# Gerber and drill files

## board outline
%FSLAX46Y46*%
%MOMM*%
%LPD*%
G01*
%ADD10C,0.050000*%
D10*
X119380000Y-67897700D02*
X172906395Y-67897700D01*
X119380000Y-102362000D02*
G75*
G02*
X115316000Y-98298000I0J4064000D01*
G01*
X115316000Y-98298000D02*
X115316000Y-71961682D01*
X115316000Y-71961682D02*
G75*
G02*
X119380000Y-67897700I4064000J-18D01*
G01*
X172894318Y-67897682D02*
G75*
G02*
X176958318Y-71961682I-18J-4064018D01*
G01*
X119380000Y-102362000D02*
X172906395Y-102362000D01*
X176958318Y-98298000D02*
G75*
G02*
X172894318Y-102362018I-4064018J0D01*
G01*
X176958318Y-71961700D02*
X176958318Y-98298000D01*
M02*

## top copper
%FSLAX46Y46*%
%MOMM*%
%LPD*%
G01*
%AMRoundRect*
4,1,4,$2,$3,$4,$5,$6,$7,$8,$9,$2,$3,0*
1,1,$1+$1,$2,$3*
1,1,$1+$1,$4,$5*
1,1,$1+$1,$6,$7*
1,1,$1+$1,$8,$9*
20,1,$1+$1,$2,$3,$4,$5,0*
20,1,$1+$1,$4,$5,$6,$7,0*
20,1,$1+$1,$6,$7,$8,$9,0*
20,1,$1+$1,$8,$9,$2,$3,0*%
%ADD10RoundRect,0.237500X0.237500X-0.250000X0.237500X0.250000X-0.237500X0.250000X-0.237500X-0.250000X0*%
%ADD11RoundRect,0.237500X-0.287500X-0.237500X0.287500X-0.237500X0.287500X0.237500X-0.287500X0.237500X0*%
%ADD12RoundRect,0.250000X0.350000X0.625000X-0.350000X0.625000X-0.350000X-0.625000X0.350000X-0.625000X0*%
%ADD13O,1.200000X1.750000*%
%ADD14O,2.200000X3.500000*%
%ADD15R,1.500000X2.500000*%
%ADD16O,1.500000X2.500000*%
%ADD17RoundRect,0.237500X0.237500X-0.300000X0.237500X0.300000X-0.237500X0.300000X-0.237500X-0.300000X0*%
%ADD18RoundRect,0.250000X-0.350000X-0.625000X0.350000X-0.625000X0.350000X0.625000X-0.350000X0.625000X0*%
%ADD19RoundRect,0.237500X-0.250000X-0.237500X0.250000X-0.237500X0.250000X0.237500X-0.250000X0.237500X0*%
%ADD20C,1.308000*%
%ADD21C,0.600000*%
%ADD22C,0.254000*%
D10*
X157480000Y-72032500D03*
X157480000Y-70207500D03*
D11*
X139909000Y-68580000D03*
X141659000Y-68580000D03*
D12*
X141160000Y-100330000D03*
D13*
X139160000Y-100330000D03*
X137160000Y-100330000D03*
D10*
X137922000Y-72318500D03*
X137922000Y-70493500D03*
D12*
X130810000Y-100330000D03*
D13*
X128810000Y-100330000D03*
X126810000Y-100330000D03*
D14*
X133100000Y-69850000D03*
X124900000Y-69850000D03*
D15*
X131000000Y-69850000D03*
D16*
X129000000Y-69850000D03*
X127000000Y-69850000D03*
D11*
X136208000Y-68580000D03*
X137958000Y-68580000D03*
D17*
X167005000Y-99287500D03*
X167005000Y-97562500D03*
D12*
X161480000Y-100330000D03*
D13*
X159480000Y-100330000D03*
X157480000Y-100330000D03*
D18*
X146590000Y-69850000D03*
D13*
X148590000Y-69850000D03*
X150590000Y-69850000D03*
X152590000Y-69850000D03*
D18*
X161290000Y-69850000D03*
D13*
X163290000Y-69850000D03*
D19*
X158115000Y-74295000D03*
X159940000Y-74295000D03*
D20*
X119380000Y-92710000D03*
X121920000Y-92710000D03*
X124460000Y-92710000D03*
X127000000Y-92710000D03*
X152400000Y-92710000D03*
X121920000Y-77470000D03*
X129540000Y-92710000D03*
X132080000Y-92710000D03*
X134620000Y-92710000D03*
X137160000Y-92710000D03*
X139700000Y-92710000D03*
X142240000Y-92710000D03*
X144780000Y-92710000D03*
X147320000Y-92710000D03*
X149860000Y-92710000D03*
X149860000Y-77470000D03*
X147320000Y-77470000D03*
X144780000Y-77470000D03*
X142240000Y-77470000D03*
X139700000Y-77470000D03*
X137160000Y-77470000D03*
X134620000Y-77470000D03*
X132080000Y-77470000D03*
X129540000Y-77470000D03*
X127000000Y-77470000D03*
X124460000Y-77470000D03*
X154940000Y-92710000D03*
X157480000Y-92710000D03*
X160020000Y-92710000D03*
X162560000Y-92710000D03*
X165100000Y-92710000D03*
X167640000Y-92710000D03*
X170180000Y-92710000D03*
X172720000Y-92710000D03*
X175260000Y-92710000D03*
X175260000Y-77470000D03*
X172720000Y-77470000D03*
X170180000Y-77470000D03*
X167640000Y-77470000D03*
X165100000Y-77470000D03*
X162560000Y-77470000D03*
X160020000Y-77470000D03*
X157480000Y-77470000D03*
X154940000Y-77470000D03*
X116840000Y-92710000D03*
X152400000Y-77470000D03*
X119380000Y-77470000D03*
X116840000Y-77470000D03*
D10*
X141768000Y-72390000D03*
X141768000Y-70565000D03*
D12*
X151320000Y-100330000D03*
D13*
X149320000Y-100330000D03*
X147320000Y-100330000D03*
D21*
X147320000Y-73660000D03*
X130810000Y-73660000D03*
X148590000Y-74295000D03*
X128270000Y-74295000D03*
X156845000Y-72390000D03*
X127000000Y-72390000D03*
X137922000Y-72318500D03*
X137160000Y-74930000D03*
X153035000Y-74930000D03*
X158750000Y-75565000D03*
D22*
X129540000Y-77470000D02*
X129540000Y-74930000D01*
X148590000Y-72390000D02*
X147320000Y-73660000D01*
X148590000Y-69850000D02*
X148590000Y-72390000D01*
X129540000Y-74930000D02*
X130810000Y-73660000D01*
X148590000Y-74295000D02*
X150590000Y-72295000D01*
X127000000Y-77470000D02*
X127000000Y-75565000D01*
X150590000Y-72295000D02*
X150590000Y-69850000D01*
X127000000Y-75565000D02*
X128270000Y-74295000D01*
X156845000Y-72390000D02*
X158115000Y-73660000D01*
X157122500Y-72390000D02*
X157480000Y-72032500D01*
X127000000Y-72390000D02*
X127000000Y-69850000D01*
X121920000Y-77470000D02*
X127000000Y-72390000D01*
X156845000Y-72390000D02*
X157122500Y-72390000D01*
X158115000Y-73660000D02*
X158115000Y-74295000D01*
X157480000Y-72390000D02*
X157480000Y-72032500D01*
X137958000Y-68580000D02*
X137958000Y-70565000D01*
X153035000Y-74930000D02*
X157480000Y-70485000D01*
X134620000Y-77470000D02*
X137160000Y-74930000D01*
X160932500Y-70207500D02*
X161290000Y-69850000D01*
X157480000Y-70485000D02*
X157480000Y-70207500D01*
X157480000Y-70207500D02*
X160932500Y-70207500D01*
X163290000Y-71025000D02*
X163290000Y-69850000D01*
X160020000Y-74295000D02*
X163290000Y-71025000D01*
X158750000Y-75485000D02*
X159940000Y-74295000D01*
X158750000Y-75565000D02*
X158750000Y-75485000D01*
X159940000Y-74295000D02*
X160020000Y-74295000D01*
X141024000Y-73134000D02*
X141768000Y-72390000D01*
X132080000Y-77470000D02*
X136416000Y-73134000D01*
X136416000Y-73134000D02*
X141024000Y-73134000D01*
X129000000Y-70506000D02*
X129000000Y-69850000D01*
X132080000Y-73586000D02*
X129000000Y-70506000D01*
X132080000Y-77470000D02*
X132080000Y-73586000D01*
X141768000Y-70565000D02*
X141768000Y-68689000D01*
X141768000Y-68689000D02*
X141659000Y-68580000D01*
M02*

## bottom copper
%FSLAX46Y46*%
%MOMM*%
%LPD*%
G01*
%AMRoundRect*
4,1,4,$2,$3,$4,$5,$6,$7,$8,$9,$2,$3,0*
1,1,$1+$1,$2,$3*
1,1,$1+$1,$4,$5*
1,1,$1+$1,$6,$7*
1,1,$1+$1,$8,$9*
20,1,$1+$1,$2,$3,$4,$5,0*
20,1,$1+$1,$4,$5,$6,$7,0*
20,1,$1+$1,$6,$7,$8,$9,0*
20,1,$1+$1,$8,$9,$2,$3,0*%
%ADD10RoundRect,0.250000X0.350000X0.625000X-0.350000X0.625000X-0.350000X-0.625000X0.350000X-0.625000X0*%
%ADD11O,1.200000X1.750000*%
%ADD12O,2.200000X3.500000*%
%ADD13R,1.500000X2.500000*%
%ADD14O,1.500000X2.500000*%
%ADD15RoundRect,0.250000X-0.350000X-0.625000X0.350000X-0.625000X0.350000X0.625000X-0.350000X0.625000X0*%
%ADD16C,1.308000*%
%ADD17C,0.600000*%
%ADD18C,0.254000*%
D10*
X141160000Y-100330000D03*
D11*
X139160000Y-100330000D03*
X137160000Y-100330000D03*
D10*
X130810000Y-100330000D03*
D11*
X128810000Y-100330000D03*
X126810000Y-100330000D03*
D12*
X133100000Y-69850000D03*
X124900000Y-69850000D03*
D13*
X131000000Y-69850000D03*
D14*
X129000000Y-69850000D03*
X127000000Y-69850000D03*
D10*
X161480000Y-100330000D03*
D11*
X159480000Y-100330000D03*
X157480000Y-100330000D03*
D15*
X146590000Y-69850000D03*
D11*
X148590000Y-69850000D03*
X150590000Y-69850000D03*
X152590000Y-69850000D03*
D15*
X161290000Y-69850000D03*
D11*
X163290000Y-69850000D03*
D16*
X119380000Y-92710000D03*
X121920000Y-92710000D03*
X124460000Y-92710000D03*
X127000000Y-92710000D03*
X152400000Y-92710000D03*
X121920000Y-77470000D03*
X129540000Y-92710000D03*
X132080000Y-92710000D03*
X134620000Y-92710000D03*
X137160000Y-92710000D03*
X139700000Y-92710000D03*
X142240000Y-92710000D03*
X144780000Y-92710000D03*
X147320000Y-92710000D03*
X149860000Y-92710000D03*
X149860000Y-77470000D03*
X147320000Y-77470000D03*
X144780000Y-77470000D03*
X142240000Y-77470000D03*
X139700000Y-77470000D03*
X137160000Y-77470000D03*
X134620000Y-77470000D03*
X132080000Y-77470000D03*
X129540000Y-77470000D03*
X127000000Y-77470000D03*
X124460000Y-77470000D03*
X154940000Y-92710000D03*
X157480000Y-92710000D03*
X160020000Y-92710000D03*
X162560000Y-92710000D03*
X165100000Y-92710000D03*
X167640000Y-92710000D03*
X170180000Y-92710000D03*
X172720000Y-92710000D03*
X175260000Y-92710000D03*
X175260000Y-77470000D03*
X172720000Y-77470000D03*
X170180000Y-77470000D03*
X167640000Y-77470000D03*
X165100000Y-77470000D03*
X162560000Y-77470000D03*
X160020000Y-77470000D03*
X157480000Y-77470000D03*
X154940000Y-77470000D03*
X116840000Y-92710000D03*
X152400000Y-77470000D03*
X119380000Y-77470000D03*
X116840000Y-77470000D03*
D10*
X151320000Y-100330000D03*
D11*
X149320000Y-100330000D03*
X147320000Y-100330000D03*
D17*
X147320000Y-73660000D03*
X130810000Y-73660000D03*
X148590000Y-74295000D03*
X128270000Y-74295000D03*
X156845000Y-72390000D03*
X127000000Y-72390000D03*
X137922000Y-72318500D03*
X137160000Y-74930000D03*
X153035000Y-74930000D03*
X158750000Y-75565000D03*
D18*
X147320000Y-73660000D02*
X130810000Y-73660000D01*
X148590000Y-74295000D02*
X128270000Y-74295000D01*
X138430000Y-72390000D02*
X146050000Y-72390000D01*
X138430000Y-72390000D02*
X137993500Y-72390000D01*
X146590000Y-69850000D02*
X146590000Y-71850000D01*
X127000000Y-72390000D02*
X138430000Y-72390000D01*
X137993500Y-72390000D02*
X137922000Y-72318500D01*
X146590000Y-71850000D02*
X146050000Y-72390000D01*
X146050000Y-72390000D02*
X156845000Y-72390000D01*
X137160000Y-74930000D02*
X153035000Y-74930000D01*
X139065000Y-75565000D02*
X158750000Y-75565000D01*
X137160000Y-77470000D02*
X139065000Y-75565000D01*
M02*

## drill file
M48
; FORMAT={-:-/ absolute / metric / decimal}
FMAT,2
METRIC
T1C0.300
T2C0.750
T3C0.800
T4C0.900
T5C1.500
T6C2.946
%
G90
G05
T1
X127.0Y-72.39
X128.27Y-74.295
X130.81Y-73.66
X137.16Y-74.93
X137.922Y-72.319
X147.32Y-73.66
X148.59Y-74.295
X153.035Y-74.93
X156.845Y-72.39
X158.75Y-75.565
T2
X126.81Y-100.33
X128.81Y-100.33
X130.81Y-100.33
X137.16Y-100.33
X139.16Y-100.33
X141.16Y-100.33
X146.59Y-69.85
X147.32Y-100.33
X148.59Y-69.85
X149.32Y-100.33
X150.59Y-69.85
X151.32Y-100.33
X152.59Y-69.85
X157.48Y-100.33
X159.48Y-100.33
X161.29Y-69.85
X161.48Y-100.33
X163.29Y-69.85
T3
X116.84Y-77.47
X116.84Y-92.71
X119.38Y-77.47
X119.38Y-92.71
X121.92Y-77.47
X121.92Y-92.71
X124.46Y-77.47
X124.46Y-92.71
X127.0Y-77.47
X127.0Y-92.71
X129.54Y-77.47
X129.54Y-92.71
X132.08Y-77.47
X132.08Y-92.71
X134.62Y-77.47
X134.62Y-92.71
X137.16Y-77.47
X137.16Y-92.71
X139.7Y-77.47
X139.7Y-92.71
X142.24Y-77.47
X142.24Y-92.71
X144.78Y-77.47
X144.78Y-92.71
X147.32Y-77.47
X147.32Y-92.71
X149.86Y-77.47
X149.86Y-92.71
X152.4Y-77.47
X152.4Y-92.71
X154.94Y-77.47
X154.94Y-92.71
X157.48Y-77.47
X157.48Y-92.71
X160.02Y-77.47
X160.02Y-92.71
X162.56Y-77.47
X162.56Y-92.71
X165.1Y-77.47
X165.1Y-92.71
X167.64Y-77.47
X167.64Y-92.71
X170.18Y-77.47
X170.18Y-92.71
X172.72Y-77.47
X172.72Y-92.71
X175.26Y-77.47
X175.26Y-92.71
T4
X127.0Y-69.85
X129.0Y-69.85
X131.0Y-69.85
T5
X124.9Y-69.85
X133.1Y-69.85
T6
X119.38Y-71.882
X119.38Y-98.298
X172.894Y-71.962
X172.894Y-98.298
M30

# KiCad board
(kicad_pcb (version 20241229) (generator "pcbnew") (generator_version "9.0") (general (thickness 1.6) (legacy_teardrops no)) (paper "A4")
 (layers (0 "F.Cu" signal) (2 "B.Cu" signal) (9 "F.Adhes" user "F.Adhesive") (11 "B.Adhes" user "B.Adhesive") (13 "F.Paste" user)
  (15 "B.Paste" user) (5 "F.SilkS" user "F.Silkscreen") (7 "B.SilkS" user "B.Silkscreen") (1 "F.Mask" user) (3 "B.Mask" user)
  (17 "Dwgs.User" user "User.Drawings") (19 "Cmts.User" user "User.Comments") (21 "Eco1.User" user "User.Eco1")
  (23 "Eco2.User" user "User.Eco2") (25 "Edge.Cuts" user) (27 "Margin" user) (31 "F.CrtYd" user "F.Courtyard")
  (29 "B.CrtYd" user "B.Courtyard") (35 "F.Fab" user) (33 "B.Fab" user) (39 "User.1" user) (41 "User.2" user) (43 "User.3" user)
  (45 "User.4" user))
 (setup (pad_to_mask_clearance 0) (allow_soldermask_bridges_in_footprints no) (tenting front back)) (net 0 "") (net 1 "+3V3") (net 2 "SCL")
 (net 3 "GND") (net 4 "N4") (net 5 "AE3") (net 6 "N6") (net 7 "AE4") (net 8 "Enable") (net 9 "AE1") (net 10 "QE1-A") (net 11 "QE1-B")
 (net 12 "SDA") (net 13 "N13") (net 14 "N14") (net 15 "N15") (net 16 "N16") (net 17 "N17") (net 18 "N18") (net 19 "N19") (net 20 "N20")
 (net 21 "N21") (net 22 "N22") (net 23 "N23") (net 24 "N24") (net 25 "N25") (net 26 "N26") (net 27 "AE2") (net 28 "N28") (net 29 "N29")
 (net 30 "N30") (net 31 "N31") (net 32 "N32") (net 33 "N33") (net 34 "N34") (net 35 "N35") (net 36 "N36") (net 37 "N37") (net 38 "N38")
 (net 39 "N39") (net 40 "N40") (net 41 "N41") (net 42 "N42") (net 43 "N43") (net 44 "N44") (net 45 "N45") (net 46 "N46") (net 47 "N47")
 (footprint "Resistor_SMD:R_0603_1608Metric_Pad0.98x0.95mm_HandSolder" (layer "F.Cu") (at 157.48 71.12 90)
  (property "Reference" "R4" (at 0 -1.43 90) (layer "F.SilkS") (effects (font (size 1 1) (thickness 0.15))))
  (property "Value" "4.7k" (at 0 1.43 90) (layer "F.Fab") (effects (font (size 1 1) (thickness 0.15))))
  (pad "1" smd roundrect (at -0.9125 0 90) (size 0.975 0.95) (layers "F.Cu" "F.Mask" "F.Paste") (roundrect_rratio 0.25) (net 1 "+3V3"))
  (pad "2" smd roundrect (at 0.9125 0 90) (size 0.975 0.95) (layers "F.Cu" "F.Mask" "F.Paste") (roundrect_rratio 0.25) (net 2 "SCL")))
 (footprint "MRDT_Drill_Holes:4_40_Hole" (layer "F.Cu") (at 172.894318 98.298)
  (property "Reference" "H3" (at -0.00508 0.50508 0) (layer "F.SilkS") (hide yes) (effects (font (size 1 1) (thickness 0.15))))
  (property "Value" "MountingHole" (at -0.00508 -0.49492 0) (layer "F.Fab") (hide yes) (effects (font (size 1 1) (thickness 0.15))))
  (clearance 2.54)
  (pad "" np_thru_hole circle (at 0 0) (size 2.9464 2.9464) (drill 2.9464) (layers "*.Cu" "*.Mask") (clearance 2.5)))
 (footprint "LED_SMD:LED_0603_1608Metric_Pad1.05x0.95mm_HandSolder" (layer "F.Cu") (at 140.784 68.58)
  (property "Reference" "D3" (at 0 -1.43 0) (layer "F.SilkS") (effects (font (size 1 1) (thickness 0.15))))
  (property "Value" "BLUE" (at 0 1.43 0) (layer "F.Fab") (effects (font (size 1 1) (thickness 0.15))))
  (pad "1" smd roundrect (at -0.875 0) (size 1.05 0.95) (layers "F.Cu" "F.Mask" "F.Paste") (roundrect_rratio 0.25) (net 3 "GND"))
  (pad "2" smd roundrect (at 0.875 0) (size 1.05 0.95) (layers "F.Cu" "F.Mask" "F.Paste") (roundrect_rratio 0.25) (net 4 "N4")))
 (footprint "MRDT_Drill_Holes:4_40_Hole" (layer "F.Cu") (at 119.38 71.882)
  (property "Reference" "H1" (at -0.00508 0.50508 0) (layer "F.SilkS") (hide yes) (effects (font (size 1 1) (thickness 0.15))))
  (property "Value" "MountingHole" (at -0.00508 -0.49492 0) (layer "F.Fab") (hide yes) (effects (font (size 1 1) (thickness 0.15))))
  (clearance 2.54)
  (pad "" np_thru_hole circle (at 0 0) (size 2.9464 2.9464) (drill 2.9464) (layers "*.Cu" "*.Mask") (clearance 2.5)))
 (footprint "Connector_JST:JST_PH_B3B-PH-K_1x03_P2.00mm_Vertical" (layer "F.Cu") (at 141.16 100.33 180)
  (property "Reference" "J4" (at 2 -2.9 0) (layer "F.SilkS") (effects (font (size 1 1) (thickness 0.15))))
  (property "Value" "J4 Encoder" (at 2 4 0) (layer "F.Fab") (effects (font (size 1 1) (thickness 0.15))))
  (pad "1" thru_hole roundrect (at 0 0 180) (size 1.2 1.75) (drill 0.75) (layers "*.Cu" "*.Mask") (remove_unused_layers no)
   (roundrect_rratio 0.208333) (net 1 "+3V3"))
  (pad "2" thru_hole oval (at 2 0 180) (size 1.2 1.75) (drill 0.75) (layers "*.Cu" "*.Mask") (remove_unused_layers no) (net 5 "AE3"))
  (pad "3" thru_hole oval (at 4 0 180) (size 1.2 1.75) (drill 0.75) (layers "*.Cu" "*.Mask") (remove_unused_layers no) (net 3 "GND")))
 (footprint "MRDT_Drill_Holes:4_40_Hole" (layer "F.Cu") (at 119.38 98.298)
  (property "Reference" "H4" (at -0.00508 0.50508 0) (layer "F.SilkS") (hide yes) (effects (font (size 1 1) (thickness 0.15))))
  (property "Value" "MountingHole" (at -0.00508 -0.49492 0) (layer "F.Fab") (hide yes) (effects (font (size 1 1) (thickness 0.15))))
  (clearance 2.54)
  (pad "" np_thru_hole circle (at 0 0) (size 2.9464 2.9464) (drill 2.9464) (layers "*.Cu" "*.Mask") (clearance 2.5)))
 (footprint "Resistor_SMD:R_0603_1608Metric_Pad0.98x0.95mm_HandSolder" (layer "F.Cu") (at 137.922 71.406 90)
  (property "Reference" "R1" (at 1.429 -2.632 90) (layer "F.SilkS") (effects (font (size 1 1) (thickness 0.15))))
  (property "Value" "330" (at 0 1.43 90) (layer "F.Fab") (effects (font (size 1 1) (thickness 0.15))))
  (pad "1" smd roundrect (at -0.9125 0 90) (size 0.975 0.95) (layers "F.Cu" "F.Mask" "F.Paste") (roundrect_rratio 0.25) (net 1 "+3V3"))
  (pad "2" smd roundrect (at 0.9125 0 90) (size 0.975 0.95) (layers "F.Cu" "F.Mask" "F.Paste") (roundrect_rratio 0.25) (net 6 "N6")))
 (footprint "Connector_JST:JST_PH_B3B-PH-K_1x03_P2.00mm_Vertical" (layer "F.Cu") (at 130.81 100.33 180)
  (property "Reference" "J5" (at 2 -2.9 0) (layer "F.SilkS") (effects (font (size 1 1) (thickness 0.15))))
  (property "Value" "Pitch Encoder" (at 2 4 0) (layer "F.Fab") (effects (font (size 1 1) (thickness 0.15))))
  (pad "1" thru_hole roundrect (at 0 0 180) (size 1.2 1.75) (drill 0.75) (layers "*.Cu" "*.Mask") (remove_unused_layers no)
   (roundrect_rratio 0.208333) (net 1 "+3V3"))
  (pad "2" thru_hole oval (at 2 0 180) (size 1.2 1.75) (drill 0.75) (layers "*.Cu" "*.Mask") (remove_unused_layers no) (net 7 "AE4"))
  (pad "3" thru_hole oval (at 4 0 180) (size 1.2 1.75) (drill 0.75) (layers "*.Cu" "*.Mask") (remove_unused_layers no) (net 3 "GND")))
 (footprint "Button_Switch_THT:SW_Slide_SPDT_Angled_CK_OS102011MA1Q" (layer "F.Cu") (at 131 69.85 180)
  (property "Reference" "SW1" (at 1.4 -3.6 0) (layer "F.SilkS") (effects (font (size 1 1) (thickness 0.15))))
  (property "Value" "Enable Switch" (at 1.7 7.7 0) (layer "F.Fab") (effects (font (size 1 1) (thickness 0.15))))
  (pad "" thru_hole oval (at -2.1 0 180) (size 2.2 3.5) (drill 1.5) (layers "*.Cu" "*.Mask") (remove_unused_layers no))
  (pad "" thru_hole oval (at 6.1 0 180) (size 2.2 3.5) (drill 1.5) (layers "*.Cu" "*.Mask") (remove_unused_layers no))
  (pad "1" thru_hole rect (at 0 0 180) (size 1.5 2.5) (drill 0.9) (layers "*.Cu" "*.Mask") (remove_unused_layers no) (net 3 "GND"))
  (pad "2" thru_hole oval (at 2 0 180) (size 1.5 2.5) (drill 0.9) (layers "*.Cu" "*.Mask") (remove_unused_layers no) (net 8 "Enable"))
  (pad "3" thru_hole oval (at 4 0 180) (size 1.5 2.5) (drill 0.9) (layers "*.Cu" "*.Mask") (remove_unused_layers no) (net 1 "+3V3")))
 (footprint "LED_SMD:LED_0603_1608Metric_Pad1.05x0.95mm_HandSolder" (layer "F.Cu") (at 137.083 68.58)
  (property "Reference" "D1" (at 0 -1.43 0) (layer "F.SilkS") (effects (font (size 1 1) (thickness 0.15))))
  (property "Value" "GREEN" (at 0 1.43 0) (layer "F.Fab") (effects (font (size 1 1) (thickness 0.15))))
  (pad "1" smd roundrect (at -0.875 0) (size 1.05 0.95) (layers "F.Cu" "F.Mask" "F.Paste") (roundrect_rratio 0.25) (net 3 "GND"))
  (pad "2" smd roundrect (at 0.875 0) (size 1.05 0.95) (layers "F.Cu" "F.Mask" "F.Paste") (roundrect_rratio 0.25) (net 6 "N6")))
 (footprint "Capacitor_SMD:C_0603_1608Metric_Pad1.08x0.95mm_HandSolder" (layer "F.Cu") (at 167.005 98.425 90)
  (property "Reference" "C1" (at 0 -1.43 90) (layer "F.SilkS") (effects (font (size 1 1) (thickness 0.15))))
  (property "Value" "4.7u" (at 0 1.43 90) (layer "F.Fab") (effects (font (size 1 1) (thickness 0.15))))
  (pad "1" smd roundrect (at -0.8625 0 90) (size 1.075 0.95) (layers "F.Cu" "F.Mask" "F.Paste") (roundrect_rratio 0.25) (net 1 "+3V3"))
  (pad "2" smd roundrect (at 0.8625 0 90) (size 1.075 0.95) (layers "F.Cu" "F.Mask" "F.Paste") (roundrect_rratio 0.25) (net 3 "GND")))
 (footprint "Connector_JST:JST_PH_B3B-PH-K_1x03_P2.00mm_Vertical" (layer "F.Cu") (at 161.48 100.33 180)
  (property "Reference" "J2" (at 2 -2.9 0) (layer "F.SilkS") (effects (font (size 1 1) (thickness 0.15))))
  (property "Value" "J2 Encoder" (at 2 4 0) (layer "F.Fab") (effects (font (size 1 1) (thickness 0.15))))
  (pad "1" thru_hole roundrect (at 0 0 180) (size 1.2 1.75) (drill 0.75) (layers "*.Cu" "*.Mask") (remove_unused_layers no)
   (roundrect_rratio 0.208333) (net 1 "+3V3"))
  (pad "2" thru_hole oval (at 2 0 180) (size 1.2 1.75) (drill 0.75) (layers "*.Cu" "*.Mask") (remove_unused_layers no) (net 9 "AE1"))
  (pad "3" thru_hole oval (at 4 0 180) (size 1.2 1.75) (drill 0.75) (layers "*.Cu" "*.Mask") (remove_unused_layers no) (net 3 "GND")))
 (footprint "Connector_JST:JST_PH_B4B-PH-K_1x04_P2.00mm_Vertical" (layer "F.Cu") (at 146.59 69.85)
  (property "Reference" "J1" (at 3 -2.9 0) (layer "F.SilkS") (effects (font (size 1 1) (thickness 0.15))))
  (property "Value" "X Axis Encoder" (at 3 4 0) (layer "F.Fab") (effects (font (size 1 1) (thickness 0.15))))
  (pad "1" thru_hole roundrect (at 0 0) (size 1.2 1.75) (drill 0.75) (layers "*.Cu" "*.Mask") (remove_unused_layers no)
   (roundrect_rratio 0.208333) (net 1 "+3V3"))
  (pad "2" thru_hole oval (at 2 0) (size 1.2 1.75) (drill 0.75) (layers "*.Cu" "*.Mask") (remove_unused_layers no) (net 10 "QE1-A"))
  (pad "3" thru_hole oval (at 4 0) (size 1.2 1.75) (drill 0.75) (layers "*.Cu" "*.Mask") (remove_unused_layers no) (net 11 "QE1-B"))
  (pad "4" thru_hole oval (at 6 0) (size 1.2 1.75) (drill 0.75) (layers "*.Cu" "*.Mask") (remove_unused_layers no) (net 3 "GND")))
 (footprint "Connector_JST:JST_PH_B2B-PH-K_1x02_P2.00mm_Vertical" (layer "F.Cu") (at 161.29 69.85)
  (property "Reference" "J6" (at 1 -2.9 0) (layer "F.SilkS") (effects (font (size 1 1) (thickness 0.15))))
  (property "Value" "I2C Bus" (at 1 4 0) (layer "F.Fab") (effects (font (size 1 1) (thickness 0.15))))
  (pad "1" thru_hole roundrect (at 0 0) (size 1.2 1.75) (drill 0.75) (layers "*.Cu" "*.Mask") (remove_unused_layers no)
   (roundrect_rratio 0.208333) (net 2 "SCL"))
  (pad "2" thru_hole oval (at 2 0) (size 1.2 1.75) (drill 0.75) (layers "*.Cu" "*.Mask") (remove_unused_layers no) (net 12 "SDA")))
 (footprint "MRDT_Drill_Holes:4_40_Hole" (layer "F.Cu") (at 172.894318 71.961682)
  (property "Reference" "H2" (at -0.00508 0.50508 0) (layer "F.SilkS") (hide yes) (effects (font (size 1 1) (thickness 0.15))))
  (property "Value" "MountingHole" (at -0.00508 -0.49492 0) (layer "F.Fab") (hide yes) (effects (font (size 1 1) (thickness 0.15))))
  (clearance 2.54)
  (pad "" np_thru_hole circle (at 0 0) (size 2.9464 2.9464) (drill 2.9464) (layers "*.Cu" "*.Mask") (clearance 2.5)))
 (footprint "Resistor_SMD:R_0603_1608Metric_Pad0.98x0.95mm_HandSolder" (layer "F.Cu") (at 159.0275 74.295)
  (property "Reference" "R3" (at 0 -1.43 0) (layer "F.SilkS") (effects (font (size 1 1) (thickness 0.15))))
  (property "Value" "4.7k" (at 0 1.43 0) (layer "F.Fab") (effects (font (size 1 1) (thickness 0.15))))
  (pad "1" smd roundrect (at -0.9125 0) (size 0.975 0.95) (layers "F.Cu" "F.Mask" "F.Paste") (roundrect_rratio 0.25) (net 1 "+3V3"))
  (pad "2" smd roundrect (at 0.9125 0) (size 0.975 0.95) (layers "F.Cu" "F.Mask" "F.Paste") (roundrect_rratio 0.25) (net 12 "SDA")))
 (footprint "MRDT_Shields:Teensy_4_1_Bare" (layer "F.Cu") (at 146.05 85.09)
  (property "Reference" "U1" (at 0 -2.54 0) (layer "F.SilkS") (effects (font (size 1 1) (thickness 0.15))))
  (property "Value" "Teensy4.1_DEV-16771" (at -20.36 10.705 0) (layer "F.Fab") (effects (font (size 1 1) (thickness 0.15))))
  (pad "0" thru_hole circle (at -26.67 7.62) (size 1.308 1.308) (drill 0.8) (layers "*.Cu" "*.Mask") (remove_unused_layers no)
   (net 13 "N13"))
  (pad "1" thru_hole circle (at -24.13 7.62) (size 1.308 1.308) (drill 0.8) (layers "*.Cu" "*.Mask") (remove_unused_layers no)
   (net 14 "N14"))
  (pad "2" thru_hole circle (at -21.59 7.62) (size 1.308 1.308) (drill 0.8) (layers "*.Cu" "*.Mask") (remove_unused_layers no)
   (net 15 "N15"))
  (pad "3" thru_hole circle (at -19.05 7.62) (size 1.308 1.308) (drill 0.8) (layers "*.Cu" "*.Mask") (remove_unused_layers no)
   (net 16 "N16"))
  (pad "3.3V_1" thru_hole circle (at 6.35 7.62) (size 1.308 1.308) (drill 0.8) (layers "*.Cu" "*.Mask") (remove_unused_layers no)
   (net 1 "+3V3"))
  (pad "3.3V_2" thru_hole circle (at -24.13 -7.62) (size 1.308 1.308) (drill 0.8) (layers "*.Cu" "*.Mask") (remove_unused_layers no)
   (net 1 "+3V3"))
  (pad "4" thru_hole circle (at -16.51 7.62) (size 1.308 1.308) (drill 0.8) (layers "*.Cu" "*.Mask") (remove_unused_layers no)
   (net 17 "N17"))
  (pad "5" thru_hole circle (at -13.97 7.62) (size 1.308 1.308) (drill 0.8) (layers "*.Cu" "*.Mask") (remove_unused_layers no)
   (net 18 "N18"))
  (pad "6" thru_hole circle (at -11.43 7.62) (size 1.308 1.308) (drill 0.8) (layers "*.Cu" "*.Mask") (remove_unused_layers no)
   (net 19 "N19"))
  (pad "7" thru_hole circle (at -8.89 7.62) (size 1.308 1.308) (drill 0.8) (layers "*.Cu" "*.Mask") (remove_unused_layers no) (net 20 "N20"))
  (pad "8" thru_hole circle (at -6.35 7.62) (size 1.308 1.308) (drill 0.8) (layers "*.Cu" "*.Mask") (remove_unused_layers no) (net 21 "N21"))
  (pad "9" thru_hole circle (at -3.81 7.62) (size 1.308 1.308) (drill 0.8) (layers "*.Cu" "*.Mask") (remove_unused_layers no) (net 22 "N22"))
  (pad "10" thru_hole circle (at -1.27 7.62) (size 1.308 1.308) (drill 0.8) (layers "*.Cu" "*.Mask") (remove_unused_layers no)
   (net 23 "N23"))
  (pad "11" thru_hole circle (at 1.27 7.62) (size 1.308 1.308) (drill 0.8) (layers "*.Cu" "*.Mask") (remove_unused_layers no) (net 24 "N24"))
  (pad "12" thru_hole circle (at 3.81 7.62) (size 1.308 1.308) (drill 0.8) (layers "*.Cu" "*.Mask") (remove_unused_layers no) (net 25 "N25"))
  (pad "13" thru_hole circle (at 3.81 -7.62) (size 1.308 1.308) (drill 0.8) (layers "*.Cu" "*.Mask") (remove_unused_layers no)
   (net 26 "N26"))
  (pad "14" thru_hole circle (at 1.27 -7.62) (size 1.308 1.308) (drill 0.8) (layers "*.Cu" "*.Mask") (remove_unused_layers no) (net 9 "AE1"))
  (pad "15" thru_hole circle (at -1.27 -7.62) (size 1.308 1.308) (drill 0.8) (layers "*.Cu" "*.Mask") (remove_unused_layers no)
   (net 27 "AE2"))
  (pad "16" thru_hole circle (at -3.81 -7.62) (size 1.308 1.308) (drill 0.8) (layers "*.Cu" "*.Mask") (remove_unused_layers no)
   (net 5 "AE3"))
  (pad "17" thru_hole circle (at -6.35 -7.62) (size 1.308 1.308) (drill 0.8) (layers "*.Cu" "*.Mask") (remove_unused_layers no)
   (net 7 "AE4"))
  (pad "18" thru_hole circle (at -8.89 -7.62) (size 1.308 1.308) (drill 0.8) (layers "*.Cu" "*.Mask") (remove_unused_layers no)
   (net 12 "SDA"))
  (pad "19" thru_hole circle (at -11.43 -7.62) (size 1.308 1.308) (drill 0.8) (layers "*.Cu" "*.Mask") (remove_unused_layers no)
   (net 2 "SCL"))
  (pad "20" thru_hole circle (at -13.97 -7.62) (size 1.308 1.308) (drill 0.8) (layers "*.Cu" "*.Mask") (remove_unused_layers no)
   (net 8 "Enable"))
  (pad "21" thru_hole circle (at -16.51 -7.62) (size 1.308 1.308) (drill 0.8) (layers "*.Cu" "*.Mask") (remove_unused_layers no)
   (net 10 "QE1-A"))
  (pad "22" thru_hole circle (at -19.05 -7.62) (size 1.308 1.308) (drill 0.8) (layers "*.Cu" "*.Mask") (remove_unused_layers no)
   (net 11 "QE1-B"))
  (pad "23" thru_hole circle (at -21.59 -7.62) (size 1.308 1.308) (drill 0.8) (layers "*.Cu" "*.Mask") (remove_unused_layers no)
   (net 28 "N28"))
  (pad "24" thru_hole circle (at 8.89 7.62) (size 1.308 1.308) (drill 0.8) (layers "*.Cu" "*.Mask") (remove_unused_layers no) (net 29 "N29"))
  (pad "25" thru_hole circle (at 11.43 7.62) (size 1.308 1.308) (drill 0.8) (layers "*.Cu" "*.Mask") (remove_unused_layers no)
   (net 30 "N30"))
  (pad "26" thru_hole circle (at 13.97 7.62) (size 1.308 1.308) (drill 0.8) (layers "*.Cu" "*.Mask") (remove_unused_layers no)
   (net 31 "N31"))
  (pad "27" thru_hole circle (at 16.51 7.62) (size 1.308 1.308) (drill 0.8) (layers "*.Cu" "*.Mask") (remove_unused_layers no)
   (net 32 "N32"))
  (pad "28" thru_hole circle (at 19.05 7.62) (size 1.308 1.308) (drill 0.8) (layers "*.Cu" "*.Mask") (remove_unused_layers no)
   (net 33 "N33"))
  (pad "29" thru_hole circle (at 21.59 7.62) (size 1.308 1.308) (drill 0.8) (layers "*.Cu" "*.Mask") (remove_unused_layers no)
   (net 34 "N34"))
  (pad "30" thru_hole circle (at 24.13 7.62) (size 1.308 1.308) (drill 0.8) (layers "*.Cu" "*.Mask") (remove_unused_layers no)
   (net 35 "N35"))
  (pad "31" thru_hole circle (at 26.67 7.62) (size 1.308 1.308) (drill 0.8) (layers "*.Cu" "*.Mask") (remove_unused_layers no)
   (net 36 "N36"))
  (pad "32" thru_hole circle (at 29.21 7.62) (size 1.308 1.308) (drill 0.8) (layers "*.Cu" "*.Mask") (remove_unused_layers no)
   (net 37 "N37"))
  (pad "33" thru_hole circle (at 29.21 -7.62) (size 1.308 1.308) (drill 0.8) (layers "*.Cu" "*.Mask") (remove_unused_layers no)
   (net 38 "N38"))
  (pad "34" thru_hole circle (at 26.67 -7.62) (size 1.308 1.308) (drill 0.8) (layers "*.Cu" "*.Mask") (remove_unused_layers no)
   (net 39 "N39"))
  (pad "35" thru_hole circle (at 24.13 -7.62) (size 1.308 1.308) (drill 0.8) (layers "*.Cu" "*.Mask") (remove_unused_layers no)
   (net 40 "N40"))
  (pad "36" thru_hole circle (at 21.59 -7.62) (size 1.308 1.308) (drill 0.8) (layers "*.Cu" "*.Mask") (remove_unused_layers no)
   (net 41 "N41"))
  (pad "37" thru_hole circle (at 19.05 -7.62) (size 1.308 1.308) (drill 0.8) (layers "*.Cu" "*.Mask") (remove_unused_layers no)
   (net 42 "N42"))
  (pad "38" thru_hole circle (at 16.51 -7.62) (size 1.308 1.308) (drill 0.8) (layers "*.Cu" "*.Mask") (remove_unused_layers no)
   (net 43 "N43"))
  (pad "39" thru_hole circle (at 13.97 -7.62) (size 1.308 1.308) (drill 0.8) (layers "*.Cu" "*.Mask") (remove_unused_layers no)
   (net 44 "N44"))
  (pad "40" thru_hole circle (at 11.43 -7.62) (size 1.308 1.308) (drill 0.8) (layers "*.Cu" "*.Mask") (remove_unused_layers no)
   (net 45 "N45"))
  (pad "41" thru_hole circle (at 8.89 -7.62) (size 1.308 1.308) (drill 0.8) (layers "*.Cu" "*.Mask") (remove_unused_layers no)
   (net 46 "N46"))
  (pad "GND1" thru_hole circle (at -29.21 7.62) (size 1.308 1.308) (drill 0.8) (layers "*.Cu" "*.Mask") (remove_unused_layers no)
   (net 3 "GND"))
  (pad "GND2" thru_hole circle (at 6.35 -7.62) (size 1.308 1.308) (drill 0.8) (layers "*.Cu" "*.Mask") (remove_unused_layers no)
   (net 3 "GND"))
  (pad "GND3" thru_hole circle (at -26.67 -7.62) (size 1.308 1.308) (drill 0.8) (layers "*.Cu" "*.Mask") (remove_unused_layers no)
   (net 3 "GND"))
  (pad "VIN" thru_hole circle (at -29.21 -7.62) (size 1.308 1.308) (drill 0.8) (layers "*.Cu" "*.Mask") (remove_unused_layers no)
   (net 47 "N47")))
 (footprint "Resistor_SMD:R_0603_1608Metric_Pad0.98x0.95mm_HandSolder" (layer "F.Cu") (at 141.768 71.4775 90)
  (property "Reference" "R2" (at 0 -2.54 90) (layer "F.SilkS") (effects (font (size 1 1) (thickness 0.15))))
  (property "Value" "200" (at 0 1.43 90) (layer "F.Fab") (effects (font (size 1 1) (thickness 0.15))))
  (pad "1" smd roundrect (at -0.9125 0 90) (size 0.975 0.95) (layers "F.Cu" "F.Mask" "F.Paste") (roundrect_rratio 0.25) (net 8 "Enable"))
  (pad "2" smd roundrect (at 0.9125 0 90) (size 0.975 0.95) (layers "F.Cu" "F.Mask" "F.Paste") (roundrect_rratio 0.25) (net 4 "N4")))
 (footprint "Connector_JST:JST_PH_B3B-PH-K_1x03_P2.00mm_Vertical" (layer "F.Cu") (at 151.32 100.33 180)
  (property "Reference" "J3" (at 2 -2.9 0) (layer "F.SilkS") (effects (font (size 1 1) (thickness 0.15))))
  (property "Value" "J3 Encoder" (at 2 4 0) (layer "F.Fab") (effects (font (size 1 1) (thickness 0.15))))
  (pad "1" thru_hole roundrect (at 0 0 180) (size 1.2 1.75) (drill 0.75) (layers "*.Cu" "*.Mask") (remove_unused_layers no)
   (roundrect_rratio 0.208333) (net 1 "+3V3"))
  (pad "2" thru_hole oval (at 2 0 180) (size 1.2 1.75) (drill 0.75) (layers "*.Cu" "*.Mask") (remove_unused_layers no) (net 27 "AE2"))
  (pad "3" thru_hole oval (at 4 0 180) (size 1.2 1.75) (drill 0.75) (layers "*.Cu" "*.Mask") (remove_unused_layers no) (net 3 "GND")))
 (gr_line (start 119.38 67.8977) (end 172.906395 67.8977) (stroke (width 0.05) (type default)) (layer "Edge.Cuts"))
 (gr_arc (start 119.38 102.362) (mid 116.506318 101.171682) (end 115.316 98.298) (stroke (width 0.05) (type default)) (layer "Edge.Cuts"))
 (gr_line (start 115.316 98.298) (end 115.316 71.961682) (stroke (width 0.05) (type default)) (layer "Edge.Cuts"))
 (gr_arc (start 115.316 71.961682) (mid 116.506318 69.088) (end 119.38 67.897682) (stroke (width 0.05) (type default)) (layer "Edge.Cuts"))
 (gr_arc (start 172.894318 67.897682) (mid 175.768 69.088) (end 176.958318 71.961682) (stroke (width 0.05) (type default))
  (layer "Edge.Cuts"))
 (gr_line (start 119.38 102.362) (end 172.906395 102.362) (stroke (width 0.05) (type default)) (layer "Edge.Cuts"))
 (gr_arc (start 176.958318 98.298) (mid 175.768 101.171682) (end 172.894318 102.362) (stroke (width 0.05) (type default))
  (layer "Edge.Cuts"))
 (gr_line (start 176.958318 71.9617) (end 176.958318 98.298) (stroke (width 0.05) (type default)) (layer "Edge.Cuts"))
 (segment (start 129.54 77.47) (end 129.54 74.93) (width 0.254) (layer "F.Cu") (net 10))
 (segment (start 148.59 72.39) (end 147.32 73.66) (width 0.254) (layer "F.Cu") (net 10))
 (segment (start 148.59 69.85) (end 148.59 72.39) (width 0.254) (layer "F.Cu") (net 10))
 (segment (start 129.54 74.93) (end 130.81 73.66) (width 0.254) (layer "F.Cu") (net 10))
 (via (at 147.32 73.66) (size 0.6) (drill 0.3) (layers "F.Cu" "B.Cu") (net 10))
 (via (at 130.81 73.66) (size 0.6) (drill 0.3) (layers "F.Cu" "B.Cu") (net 10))
 (segment (start 147.32 73.66) (end 130.81 73.66) (width 0.254) (layer "B.Cu") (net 10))
 (segment (start 148.59 74.295) (end 150.59 72.295) (width 0.254) (layer "F.Cu") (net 11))
 (segment (start 127 77.47) (end 127 75.565) (width 0.254) (layer "F.Cu") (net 11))
 (segment (start 150.59 72.295) (end 150.59 69.85) (width 0.254) (layer "F.Cu") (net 11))
 (segment (start 127 75.565) (end 128.27 74.295) (width 0.254) (layer "F.Cu") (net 11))
 (via (at 148.59 74.295) (size 0.6) (drill 0.3) (layers "F.Cu" "B.Cu") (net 11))
 (via (at 128.27 74.295) (size 0.6) (drill 0.3) (layers "F.Cu" "B.Cu") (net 11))
 (segment (start 148.59 74.295) (end 128.27 74.295) (width 0.254) (layer "B.Cu") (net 11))
 (segment (start 156.845 72.39) (end 158.115 73.66) (width 0.254) (layer "F.Cu") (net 1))
 (segment (start 157.1225 72.39) (end 157.48 72.0325) (width 0.254) (layer "F.Cu") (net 1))
 (segment (start 127 72.39) (end 127 69.85) (width 0.254) (layer "F.Cu") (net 1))
 (segment (start 121.92 77.47) (end 127 72.39) (width 0.254) (layer "F.Cu") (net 1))
 (segment (start 156.845 72.39) (end 157.1225 72.39) (width 0.254) (layer "F.Cu") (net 1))
 (segment (start 158.115 73.66) (end 158.115 74.295) (width 0.254) (layer "F.Cu") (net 1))
 (segment (start 157.48 72.39) (end 157.48 72.0325) (width 0.254) (layer "F.Cu") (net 1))
 (via (at 156.845 72.39) (size 0.6) (drill 0.3) (layers "F.Cu" "B.Cu") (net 1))
 (via (at 127 72.39) (size 0.6) (drill 0.3) (layers "F.Cu" "B.Cu") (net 1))
 (via (at 137.922 72.3185) (size 0.6) (drill 0.3) (layers "F.Cu" "B.Cu") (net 1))
 (segment (start 138.43 72.39) (end 146.05 72.39) (width 0.254) (layer "B.Cu") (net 1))
 (segment (start 138.43 72.39) (end 137.9935 72.39) (width 0.254) (layer "B.Cu") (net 1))
 (segment (start 146.59 69.85) (end 146.59 71.85) (width 0.254) (layer "B.Cu") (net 1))
 (segment (start 127 72.39) (end 138.43 72.39) (width 0.254) (layer "B.Cu") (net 1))
 (segment (start 137.9935 72.39) (end 137.922 72.3185) (width 0.254) (layer "B.Cu") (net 1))
 (segment (start 146.59 71.85) (end 146.05 72.39) (width 0.254) (layer "B.Cu") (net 1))
 (segment (start 146.05 72.39) (end 156.845 72.39) (width 0.254) (layer "B.Cu") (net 1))
 (segment (start 137.958 68.58) (end 137.958 70.565) (width 0.254) (layer "F.Cu") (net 6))
 (segment (start 153.035 74.93) (end 157.48 70.485) (width 0.254) (layer "F.Cu") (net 2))
 (segment (start 134.62 77.47) (end 137.16 74.93) (width 0.254) (layer "F.Cu") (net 2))
 (segment (start 160.9325 70.2075) (end 161.29 69.85) (width 0.254) (layer "F.Cu") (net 2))
 (segment (start 157.48 70.485) (end 157.48 70.2075) (width 0.254) (layer "F.Cu") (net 2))
 (segment (start 157.48 70.2075) (end 160.9325 70.2075) (width 0.254) (layer "F.Cu") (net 2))
 (via (at 137.16 74.93) (size 0.6) (drill 0.3) (layers "F.Cu" "B.Cu") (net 2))
 (via (at 153.035 74.93) (size 0.6) (drill 0.3) (layers "F.Cu" "B.Cu") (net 2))
 (segment (start 137.16 74.93) (end 153.035 74.93) (width 0.254) (layer "B.Cu") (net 2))
 (segment (start 163.29 71.025) (end 163.29 69.85) (width 0.254) (layer "F.Cu") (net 12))
 (segment (start 160.02 74.295) (end 163.29 71.025) (width 0.254) (layer "F.Cu") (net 12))
 (segment (start 158.75 75.485) (end 159.94 74.295) (width 0.254) (layer "F.Cu") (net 12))
 (segment (start 158.75 75.565) (end 158.75 75.485) (width 0.254) (layer "F.Cu") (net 12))
 (segment (start 159.94 74.295) (end 160.02 74.295) (width 0.254) (layer "F.Cu") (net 12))
 (via (at 158.75 75.565) (size 0.6) (drill 0.3) (layers "F.Cu" "B.Cu") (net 12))
 (segment (start 139.065 75.565) (end 158.75 75.565) (width 0.254) (layer "B.Cu") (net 12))
 (segment (start 137.16 77.47) (end 139.065 75.565) (width 0.254) (layer "B.Cu") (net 12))
 (segment (start 141.024 73.134) (end 141.768 72.39) (width 0.254) (layer "F.Cu") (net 8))
 (segment (start 132.08 77.47) (end 136.416 73.134) (width 0.254) (layer "F.Cu") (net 8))
 (segment (start 136.416 73.134) (end 141.024 73.134) (width 0.254) (layer "F.Cu") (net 8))
 (segment (start 129 70.506) (end 129 69.85) (width 0.254) (layer "F.Cu") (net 8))
 (segment (start 132.08 73.586) (end 129 70.506) (width 0.254) (layer "F.Cu") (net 8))
 (segment (start 132.08 77.47) (end 132.08 73.586) (width 0.254) (layer "F.Cu") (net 8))
 (segment (start 141.768 70.565) (end 141.768 68.689) (width 0.254) (layer "F.Cu") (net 4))
 (segment (start 141.768 68.689) (end 141.659 68.58) (width 0.254) (layer "F.Cu") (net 4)))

